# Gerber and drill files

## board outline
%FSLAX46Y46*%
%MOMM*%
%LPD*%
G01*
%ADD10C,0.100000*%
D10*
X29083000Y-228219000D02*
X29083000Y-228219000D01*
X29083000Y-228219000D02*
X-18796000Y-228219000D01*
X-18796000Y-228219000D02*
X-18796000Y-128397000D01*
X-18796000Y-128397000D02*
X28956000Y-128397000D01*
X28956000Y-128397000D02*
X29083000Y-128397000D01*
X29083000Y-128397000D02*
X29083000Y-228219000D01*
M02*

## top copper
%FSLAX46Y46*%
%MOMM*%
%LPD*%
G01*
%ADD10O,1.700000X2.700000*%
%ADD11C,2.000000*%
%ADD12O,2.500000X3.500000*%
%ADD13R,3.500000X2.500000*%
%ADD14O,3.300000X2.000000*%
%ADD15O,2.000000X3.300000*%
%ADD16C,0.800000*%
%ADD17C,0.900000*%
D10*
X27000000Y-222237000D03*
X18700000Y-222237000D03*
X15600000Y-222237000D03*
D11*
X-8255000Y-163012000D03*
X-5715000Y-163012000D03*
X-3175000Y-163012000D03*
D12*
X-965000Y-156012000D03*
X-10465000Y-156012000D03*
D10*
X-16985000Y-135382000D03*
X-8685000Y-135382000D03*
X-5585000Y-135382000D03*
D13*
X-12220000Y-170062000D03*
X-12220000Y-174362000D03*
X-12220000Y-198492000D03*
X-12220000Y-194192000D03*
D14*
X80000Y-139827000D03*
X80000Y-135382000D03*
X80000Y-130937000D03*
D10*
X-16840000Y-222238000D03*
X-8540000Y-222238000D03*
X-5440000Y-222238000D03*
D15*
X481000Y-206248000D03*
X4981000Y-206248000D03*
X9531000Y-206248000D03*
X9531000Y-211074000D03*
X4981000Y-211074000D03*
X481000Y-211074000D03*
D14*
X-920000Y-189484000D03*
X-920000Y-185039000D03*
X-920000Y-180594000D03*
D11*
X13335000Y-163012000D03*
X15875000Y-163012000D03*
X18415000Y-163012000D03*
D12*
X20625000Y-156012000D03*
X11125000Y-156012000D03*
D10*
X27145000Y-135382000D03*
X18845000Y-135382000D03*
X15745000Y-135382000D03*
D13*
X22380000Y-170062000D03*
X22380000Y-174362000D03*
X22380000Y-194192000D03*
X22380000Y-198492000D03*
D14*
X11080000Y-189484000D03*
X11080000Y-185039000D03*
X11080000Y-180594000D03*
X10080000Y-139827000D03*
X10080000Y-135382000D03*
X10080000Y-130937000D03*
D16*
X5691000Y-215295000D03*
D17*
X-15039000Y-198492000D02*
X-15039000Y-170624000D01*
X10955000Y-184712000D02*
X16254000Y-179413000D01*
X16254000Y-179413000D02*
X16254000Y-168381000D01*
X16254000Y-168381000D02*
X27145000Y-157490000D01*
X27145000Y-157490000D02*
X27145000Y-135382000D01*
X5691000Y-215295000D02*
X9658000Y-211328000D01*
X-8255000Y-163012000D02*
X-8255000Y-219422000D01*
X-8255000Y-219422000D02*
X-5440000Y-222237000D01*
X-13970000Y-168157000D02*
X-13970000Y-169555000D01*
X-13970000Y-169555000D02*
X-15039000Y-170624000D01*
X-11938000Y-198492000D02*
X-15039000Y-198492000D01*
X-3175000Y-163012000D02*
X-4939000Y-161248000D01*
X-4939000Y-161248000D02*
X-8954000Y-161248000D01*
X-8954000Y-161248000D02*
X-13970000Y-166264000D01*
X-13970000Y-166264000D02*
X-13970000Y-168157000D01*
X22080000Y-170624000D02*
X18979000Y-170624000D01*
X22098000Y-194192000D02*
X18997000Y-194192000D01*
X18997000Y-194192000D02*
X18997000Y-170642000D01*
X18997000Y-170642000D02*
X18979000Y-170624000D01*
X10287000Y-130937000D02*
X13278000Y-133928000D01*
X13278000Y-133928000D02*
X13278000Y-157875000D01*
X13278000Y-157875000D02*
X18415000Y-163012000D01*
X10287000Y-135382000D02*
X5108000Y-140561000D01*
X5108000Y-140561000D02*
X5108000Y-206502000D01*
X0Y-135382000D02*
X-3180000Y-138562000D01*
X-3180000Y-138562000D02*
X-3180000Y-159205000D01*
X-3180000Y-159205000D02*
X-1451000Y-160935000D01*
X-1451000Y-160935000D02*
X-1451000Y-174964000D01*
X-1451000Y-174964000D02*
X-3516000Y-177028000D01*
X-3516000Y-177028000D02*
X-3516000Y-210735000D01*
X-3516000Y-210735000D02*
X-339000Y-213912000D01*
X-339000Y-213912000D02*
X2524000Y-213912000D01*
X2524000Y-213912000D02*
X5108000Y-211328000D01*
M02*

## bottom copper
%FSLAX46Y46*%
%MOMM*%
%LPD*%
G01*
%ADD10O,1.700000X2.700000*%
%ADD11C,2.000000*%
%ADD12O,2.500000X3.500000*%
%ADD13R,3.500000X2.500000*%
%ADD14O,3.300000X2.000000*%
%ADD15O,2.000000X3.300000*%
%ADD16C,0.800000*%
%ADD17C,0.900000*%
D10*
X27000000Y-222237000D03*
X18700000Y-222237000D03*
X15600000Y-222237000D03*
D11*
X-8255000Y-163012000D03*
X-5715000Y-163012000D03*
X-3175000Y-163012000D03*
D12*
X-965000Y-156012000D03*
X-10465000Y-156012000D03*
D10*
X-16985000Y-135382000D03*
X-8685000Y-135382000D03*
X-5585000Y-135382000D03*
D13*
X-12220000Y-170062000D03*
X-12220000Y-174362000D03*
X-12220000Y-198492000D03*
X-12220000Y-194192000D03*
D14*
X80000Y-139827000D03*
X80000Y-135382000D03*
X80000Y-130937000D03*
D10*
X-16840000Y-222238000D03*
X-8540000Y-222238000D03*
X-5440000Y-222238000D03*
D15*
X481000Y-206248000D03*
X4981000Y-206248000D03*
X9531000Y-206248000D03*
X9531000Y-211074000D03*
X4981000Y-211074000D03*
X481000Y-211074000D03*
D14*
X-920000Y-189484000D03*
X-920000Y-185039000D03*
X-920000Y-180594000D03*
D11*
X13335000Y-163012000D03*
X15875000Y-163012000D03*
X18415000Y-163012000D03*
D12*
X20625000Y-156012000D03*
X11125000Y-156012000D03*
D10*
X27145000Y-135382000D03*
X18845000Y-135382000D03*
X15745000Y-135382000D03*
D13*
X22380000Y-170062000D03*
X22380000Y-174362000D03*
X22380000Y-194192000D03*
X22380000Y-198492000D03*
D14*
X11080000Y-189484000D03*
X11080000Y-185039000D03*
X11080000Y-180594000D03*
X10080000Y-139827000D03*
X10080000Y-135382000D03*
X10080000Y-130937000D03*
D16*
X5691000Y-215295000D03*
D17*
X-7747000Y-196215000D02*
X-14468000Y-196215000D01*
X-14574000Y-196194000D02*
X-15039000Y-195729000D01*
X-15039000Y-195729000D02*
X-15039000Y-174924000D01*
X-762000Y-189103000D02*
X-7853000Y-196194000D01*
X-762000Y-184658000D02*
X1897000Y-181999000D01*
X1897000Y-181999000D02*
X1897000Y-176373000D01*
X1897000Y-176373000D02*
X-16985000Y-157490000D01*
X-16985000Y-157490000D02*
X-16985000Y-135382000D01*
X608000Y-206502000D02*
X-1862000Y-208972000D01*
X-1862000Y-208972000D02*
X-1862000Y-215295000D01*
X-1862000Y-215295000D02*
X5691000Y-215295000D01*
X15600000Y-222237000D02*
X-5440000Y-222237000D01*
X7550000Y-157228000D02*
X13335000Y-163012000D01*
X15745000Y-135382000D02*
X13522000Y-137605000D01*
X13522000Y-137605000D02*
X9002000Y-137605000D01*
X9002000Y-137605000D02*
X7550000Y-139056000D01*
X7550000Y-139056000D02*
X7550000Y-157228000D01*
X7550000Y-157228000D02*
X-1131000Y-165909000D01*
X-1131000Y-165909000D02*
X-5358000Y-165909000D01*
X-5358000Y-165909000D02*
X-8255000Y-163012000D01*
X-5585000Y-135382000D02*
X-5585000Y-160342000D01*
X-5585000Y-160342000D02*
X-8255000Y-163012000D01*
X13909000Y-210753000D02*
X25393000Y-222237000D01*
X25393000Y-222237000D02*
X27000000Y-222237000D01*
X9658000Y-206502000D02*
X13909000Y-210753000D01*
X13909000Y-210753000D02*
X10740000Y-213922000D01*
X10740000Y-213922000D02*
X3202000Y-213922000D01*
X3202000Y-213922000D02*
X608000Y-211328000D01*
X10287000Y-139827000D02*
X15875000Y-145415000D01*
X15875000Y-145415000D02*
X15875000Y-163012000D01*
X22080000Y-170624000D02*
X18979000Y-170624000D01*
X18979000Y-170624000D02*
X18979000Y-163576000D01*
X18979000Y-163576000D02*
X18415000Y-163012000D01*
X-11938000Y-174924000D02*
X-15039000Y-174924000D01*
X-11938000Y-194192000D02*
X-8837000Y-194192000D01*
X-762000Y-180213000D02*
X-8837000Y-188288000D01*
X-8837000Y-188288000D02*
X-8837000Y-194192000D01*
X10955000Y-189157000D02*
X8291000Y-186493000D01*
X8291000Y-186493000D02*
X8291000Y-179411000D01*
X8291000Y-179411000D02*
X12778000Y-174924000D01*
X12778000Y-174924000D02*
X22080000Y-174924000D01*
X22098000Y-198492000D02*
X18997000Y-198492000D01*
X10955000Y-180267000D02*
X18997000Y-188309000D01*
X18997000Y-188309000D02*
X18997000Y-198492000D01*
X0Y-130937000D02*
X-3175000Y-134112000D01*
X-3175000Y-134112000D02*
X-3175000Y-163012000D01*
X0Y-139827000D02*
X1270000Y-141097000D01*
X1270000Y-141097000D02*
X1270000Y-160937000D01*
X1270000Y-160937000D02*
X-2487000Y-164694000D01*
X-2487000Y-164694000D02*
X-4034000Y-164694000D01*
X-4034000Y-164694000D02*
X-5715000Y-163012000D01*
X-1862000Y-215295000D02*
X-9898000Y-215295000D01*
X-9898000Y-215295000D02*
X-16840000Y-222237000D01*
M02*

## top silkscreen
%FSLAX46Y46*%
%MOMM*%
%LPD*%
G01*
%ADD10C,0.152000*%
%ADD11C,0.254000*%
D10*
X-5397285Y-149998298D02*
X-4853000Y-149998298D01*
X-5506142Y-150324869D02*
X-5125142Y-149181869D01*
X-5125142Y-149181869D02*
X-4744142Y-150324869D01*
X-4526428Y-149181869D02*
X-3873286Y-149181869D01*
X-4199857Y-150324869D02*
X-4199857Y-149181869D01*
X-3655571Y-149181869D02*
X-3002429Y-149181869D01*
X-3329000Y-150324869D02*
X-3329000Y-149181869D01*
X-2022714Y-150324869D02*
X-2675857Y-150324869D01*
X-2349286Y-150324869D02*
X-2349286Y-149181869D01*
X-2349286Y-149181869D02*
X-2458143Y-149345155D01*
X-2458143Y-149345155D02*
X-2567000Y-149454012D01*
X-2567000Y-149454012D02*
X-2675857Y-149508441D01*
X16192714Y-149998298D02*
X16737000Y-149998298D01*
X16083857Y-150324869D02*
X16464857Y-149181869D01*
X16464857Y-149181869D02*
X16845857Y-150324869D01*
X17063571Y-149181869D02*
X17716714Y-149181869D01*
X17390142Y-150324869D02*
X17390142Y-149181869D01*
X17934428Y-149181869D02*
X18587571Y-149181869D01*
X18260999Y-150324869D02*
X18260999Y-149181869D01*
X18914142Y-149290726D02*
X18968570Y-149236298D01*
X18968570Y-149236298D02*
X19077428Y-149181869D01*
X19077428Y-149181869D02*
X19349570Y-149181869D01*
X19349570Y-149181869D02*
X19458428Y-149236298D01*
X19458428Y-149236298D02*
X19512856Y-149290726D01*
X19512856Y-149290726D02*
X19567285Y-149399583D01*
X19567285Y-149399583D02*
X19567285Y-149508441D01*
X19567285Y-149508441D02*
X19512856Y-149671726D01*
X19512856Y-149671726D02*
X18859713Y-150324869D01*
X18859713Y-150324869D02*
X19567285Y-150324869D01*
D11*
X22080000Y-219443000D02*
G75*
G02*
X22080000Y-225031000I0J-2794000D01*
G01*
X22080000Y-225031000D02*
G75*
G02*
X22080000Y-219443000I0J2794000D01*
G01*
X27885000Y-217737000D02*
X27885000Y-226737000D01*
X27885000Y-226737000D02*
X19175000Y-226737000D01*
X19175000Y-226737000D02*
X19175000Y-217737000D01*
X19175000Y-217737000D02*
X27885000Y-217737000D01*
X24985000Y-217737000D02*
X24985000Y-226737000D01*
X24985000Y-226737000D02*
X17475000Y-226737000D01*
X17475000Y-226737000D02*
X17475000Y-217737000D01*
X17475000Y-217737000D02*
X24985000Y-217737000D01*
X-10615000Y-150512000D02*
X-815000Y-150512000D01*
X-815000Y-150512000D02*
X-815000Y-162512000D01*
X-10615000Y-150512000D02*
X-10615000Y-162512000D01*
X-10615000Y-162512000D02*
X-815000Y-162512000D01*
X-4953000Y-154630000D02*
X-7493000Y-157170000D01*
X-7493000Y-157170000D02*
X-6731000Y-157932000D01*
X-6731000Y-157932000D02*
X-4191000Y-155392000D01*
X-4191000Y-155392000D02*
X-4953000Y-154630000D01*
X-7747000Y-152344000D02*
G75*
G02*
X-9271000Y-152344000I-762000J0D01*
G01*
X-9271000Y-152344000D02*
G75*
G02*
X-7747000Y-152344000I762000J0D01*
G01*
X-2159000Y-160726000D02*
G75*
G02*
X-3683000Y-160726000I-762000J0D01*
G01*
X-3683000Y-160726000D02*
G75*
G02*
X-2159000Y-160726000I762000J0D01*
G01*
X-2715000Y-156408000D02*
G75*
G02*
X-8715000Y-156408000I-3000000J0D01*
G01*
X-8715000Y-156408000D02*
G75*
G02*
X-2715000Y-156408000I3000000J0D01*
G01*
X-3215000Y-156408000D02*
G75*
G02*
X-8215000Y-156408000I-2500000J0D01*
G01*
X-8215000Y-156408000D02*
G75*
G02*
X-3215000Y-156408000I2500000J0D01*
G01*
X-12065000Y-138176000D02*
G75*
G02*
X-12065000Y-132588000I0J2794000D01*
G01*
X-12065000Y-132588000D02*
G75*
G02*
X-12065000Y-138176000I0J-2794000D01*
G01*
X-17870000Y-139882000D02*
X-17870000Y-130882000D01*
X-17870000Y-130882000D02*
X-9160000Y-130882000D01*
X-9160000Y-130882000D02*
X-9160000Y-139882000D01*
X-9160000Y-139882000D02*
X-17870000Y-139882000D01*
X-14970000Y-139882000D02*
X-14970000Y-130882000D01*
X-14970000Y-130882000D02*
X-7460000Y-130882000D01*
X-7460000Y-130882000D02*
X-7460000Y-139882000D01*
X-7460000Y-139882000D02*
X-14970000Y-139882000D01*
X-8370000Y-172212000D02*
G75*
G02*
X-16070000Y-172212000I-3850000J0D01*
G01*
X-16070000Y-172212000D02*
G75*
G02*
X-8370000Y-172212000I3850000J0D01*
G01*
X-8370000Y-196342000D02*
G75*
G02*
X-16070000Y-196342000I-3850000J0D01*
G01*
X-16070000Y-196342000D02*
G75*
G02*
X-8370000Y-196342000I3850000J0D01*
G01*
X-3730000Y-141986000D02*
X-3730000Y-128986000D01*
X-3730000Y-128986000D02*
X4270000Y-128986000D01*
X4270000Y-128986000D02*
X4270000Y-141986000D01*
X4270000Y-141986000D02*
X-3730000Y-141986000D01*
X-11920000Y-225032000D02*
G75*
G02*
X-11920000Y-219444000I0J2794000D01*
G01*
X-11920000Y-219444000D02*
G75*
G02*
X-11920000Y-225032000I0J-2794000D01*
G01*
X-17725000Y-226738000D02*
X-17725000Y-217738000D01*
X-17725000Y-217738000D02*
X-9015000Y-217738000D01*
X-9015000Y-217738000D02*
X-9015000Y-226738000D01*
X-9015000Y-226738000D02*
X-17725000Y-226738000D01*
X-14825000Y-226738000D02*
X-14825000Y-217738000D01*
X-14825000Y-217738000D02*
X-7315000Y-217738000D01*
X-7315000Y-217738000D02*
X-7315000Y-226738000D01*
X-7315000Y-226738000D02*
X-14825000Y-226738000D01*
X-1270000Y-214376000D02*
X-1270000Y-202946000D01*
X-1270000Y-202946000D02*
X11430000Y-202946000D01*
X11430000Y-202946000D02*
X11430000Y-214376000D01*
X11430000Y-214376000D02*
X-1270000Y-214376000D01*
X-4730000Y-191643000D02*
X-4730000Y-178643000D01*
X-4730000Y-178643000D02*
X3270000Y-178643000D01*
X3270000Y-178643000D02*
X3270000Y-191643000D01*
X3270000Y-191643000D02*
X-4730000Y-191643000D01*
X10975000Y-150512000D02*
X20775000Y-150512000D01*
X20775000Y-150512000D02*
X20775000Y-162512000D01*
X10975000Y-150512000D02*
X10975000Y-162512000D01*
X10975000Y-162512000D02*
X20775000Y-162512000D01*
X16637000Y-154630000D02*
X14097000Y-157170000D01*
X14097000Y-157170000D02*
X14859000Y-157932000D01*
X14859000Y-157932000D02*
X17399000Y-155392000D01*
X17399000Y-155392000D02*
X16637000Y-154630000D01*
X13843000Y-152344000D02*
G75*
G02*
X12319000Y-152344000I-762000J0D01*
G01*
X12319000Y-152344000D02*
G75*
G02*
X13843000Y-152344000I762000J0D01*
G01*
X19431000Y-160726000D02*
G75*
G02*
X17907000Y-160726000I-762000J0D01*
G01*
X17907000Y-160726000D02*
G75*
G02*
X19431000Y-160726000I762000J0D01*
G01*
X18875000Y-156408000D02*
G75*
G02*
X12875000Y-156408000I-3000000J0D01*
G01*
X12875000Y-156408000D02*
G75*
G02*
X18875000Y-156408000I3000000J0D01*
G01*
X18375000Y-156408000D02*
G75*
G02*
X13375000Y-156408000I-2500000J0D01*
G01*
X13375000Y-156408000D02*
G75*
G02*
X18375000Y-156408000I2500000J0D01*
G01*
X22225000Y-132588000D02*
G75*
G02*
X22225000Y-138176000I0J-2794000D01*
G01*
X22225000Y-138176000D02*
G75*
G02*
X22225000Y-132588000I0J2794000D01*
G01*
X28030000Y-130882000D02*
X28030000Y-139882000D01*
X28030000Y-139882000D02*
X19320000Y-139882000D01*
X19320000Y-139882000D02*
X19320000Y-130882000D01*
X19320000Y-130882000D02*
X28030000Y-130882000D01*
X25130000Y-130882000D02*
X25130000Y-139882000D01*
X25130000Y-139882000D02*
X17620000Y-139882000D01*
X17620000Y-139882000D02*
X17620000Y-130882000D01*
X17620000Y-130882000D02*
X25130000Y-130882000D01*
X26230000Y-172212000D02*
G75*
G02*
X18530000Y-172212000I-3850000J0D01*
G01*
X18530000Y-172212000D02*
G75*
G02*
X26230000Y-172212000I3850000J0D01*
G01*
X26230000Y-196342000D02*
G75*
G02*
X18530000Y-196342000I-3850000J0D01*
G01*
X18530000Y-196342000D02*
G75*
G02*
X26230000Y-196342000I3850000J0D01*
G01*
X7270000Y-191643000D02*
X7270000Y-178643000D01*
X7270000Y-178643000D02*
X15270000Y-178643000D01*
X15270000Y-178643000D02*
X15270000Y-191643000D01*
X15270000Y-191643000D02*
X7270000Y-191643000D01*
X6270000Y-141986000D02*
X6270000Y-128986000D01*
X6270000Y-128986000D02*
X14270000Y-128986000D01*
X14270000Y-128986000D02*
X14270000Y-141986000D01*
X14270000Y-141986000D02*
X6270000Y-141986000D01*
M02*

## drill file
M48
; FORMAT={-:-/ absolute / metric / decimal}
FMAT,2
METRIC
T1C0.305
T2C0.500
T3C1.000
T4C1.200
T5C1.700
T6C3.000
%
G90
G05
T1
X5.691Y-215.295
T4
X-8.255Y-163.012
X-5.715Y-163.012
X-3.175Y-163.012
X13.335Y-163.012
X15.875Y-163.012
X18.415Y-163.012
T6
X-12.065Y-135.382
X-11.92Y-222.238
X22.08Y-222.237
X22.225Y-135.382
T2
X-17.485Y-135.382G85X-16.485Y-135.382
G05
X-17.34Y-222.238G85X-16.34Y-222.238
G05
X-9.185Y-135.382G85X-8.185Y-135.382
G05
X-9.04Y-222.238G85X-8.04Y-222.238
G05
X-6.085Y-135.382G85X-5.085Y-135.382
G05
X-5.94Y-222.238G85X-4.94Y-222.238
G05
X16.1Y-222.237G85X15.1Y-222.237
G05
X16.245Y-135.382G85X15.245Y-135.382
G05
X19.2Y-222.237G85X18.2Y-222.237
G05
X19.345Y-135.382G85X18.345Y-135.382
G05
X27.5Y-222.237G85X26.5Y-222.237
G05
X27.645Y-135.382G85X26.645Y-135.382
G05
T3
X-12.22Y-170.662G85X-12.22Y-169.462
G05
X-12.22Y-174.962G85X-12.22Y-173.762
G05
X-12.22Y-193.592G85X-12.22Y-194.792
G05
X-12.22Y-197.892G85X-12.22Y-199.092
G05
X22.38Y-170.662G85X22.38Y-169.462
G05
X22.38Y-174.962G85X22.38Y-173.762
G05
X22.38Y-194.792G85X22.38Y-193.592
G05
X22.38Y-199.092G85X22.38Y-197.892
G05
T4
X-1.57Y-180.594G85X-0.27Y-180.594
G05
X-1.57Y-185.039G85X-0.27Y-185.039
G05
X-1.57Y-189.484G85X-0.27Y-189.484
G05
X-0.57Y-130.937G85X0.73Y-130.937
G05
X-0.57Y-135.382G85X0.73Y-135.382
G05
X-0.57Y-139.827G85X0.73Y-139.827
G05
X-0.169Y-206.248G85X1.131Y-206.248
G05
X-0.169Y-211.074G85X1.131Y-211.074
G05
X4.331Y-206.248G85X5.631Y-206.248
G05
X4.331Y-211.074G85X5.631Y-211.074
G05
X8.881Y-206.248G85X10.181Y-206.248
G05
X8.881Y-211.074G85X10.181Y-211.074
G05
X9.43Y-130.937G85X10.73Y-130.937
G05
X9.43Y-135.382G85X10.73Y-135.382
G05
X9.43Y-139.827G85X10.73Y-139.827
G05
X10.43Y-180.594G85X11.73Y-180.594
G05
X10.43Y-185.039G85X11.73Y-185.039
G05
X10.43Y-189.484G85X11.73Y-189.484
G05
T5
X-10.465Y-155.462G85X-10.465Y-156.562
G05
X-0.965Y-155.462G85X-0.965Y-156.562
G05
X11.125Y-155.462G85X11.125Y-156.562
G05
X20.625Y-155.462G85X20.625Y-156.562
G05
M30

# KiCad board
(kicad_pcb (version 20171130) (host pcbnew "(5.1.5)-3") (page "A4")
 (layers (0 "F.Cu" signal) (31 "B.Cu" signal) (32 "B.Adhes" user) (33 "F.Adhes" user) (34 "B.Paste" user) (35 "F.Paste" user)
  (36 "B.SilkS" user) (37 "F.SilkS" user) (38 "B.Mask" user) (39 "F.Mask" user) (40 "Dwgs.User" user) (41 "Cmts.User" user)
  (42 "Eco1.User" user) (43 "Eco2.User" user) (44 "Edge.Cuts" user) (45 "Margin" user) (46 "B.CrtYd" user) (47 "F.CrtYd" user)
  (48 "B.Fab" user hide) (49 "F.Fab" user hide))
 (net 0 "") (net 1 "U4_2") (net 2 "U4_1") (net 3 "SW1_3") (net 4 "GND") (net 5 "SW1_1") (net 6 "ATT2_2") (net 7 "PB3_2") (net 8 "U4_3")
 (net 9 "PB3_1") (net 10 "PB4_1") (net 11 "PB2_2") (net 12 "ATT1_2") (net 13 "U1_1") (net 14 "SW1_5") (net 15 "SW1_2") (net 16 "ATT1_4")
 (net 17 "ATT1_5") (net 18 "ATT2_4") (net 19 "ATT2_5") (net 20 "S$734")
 (segment (start -7.747 196.215) (end -14.468 196.215) (width 0.9) (layer "B.Cu") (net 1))
 (segment (start -14.574 196.194) (end -15.039 195.729) (width 0.9) (layer "B.Cu") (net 1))
 (segment (start -15.039 195.729) (end -15.039 174.924) (width 0.9) (layer "B.Cu") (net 1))
 (segment (start -0.762 189.103) (end -7.853 196.194) (width 0.9) (layer "B.Cu") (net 1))
 (segment (start -0.762 184.658) (end 1.897 181.999) (width 0.9) (layer "B.Cu") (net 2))
 (segment (start 1.897 181.999) (end 1.897 176.373) (width 0.9) (layer "B.Cu") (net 2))
 (segment (start 1.897 176.373) (end -16.985 157.49) (width 0.9) (layer "B.Cu") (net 2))
 (segment (start -16.985 157.49) (end -16.985 135.382) (width 0.9) (layer "B.Cu") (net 2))
 (segment (start 0.608 206.502) (end -1.862 208.972) (width 0.9) (layer "B.Cu") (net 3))
 (segment (start -1.862 208.972) (end -1.862 215.295) (width 0.9) (layer "B.Cu") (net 3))
 (segment (start -1.862 215.295) (end 5.691 215.295) (width 0.9) (layer "B.Cu") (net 3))
 (segment (start 15.6 222.237) (end -5.44 222.237) (width 0.9) (layer "B.Cu") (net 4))
 (segment (start 7.55 157.228) (end 13.335 163.012) (width 0.9) (layer "B.Cu") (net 4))
 (segment (start 15.745 135.382) (end 13.522 137.605) (width 0.9) (layer "B.Cu") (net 4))
 (segment (start 13.522 137.605) (end 9.002 137.605) (width 0.9) (layer "B.Cu") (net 4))
 (segment (start 9.002 137.605) (end 7.55 139.056) (width 0.9) (layer "B.Cu") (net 4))
 (segment (start 7.55 139.056) (end 7.55 157.228) (width 0.9) (layer "B.Cu") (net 4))
 (segment (start 7.55 157.228) (end -1.131 165.909) (width 0.9) (layer "B.Cu") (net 4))
 (segment (start -1.131 165.909) (end -5.358 165.909) (width 0.9) (layer "B.Cu") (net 4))
 (segment (start -5.358 165.909) (end -8.255 163.012) (width 0.9) (layer "B.Cu") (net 4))
 (segment (start -5.585 135.382) (end -5.585 160.342) (width 0.9) (layer "B.Cu") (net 4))
 (segment (start -5.585 160.342) (end -8.255 163.012) (width 0.9) (layer "B.Cu") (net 4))
 (segment (start 13.909 210.753) (end 25.393 222.237) (width 0.9) (layer "B.Cu") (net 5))
 (segment (start 25.393 222.237) (end 27 222.237) (width 0.9) (layer "B.Cu") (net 5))
 (segment (start 9.658 206.502) (end 13.909 210.753) (width 0.9) (layer "B.Cu") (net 5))
 (segment (start 13.909 210.753) (end 10.74 213.922) (width 0.9) (layer "B.Cu") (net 5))
 (segment (start 10.74 213.922) (end 3.202 213.922) (width 0.9) (layer "B.Cu") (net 5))
 (segment (start 3.202 213.922) (end 0.608 211.328) (width 0.9) (layer "B.Cu") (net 5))
 (segment (start 10.287 139.827) (end 15.875 145.415) (width 0.9) (layer "B.Cu") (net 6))
 (segment (start 15.875 145.415) (end 15.875 163.012) (width 0.9) (layer "B.Cu") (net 6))
 (segment (start 22.08 170.624) (end 18.979 170.624) (width 0.9) (layer "B.Cu") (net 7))
 (segment (start 18.979 170.624) (end 18.979 163.576) (width 0.9) (layer "B.Cu") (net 7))
 (segment (start 18.979 163.576) (end 18.415 163.012) (width 0.9) (layer "B.Cu") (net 7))
 (segment (start -11.938 174.924) (end -15.039 174.924) (width 0.9) (layer "B.Cu") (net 1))
 (segment (start -11.938 194.192) (end -8.837 194.192) (width 0.9) (layer "B.Cu") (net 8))
 (segment (start -0.762 180.213) (end -8.837 188.288) (width 0.9) (layer "B.Cu") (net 8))
 (segment (start -8.837 188.288) (end -8.837 194.192) (width 0.9) (layer "B.Cu") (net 8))
 (segment (start 10.955 189.157) (end 8.291 186.493) (width 0.9) (layer "B.Cu") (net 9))
 (segment (start 8.291 186.493) (end 8.291 179.411) (width 0.9) (layer "B.Cu") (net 9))
 (segment (start 8.291 179.411) (end 12.778 174.924) (width 0.9) (layer "B.Cu") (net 9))
 (segment (start 12.778 174.924) (end 22.08 174.924) (width 0.9) (layer "B.Cu") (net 9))
 (segment (start 22.098 198.492) (end 18.997 198.492) (width 0.9) (layer "B.Cu") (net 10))
 (segment (start 10.955 180.267) (end 18.997 188.309) (width 0.9) (layer "B.Cu") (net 10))
 (segment (start 18.997 188.309) (end 18.997 198.492) (width 0.9) (layer "B.Cu") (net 10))
 (segment (start 0 130.937) (end -3.175 134.112) (width 0.9) (layer "B.Cu") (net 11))
 (segment (start -3.175 134.112) (end -3.175 163.012) (width 0.9) (layer "B.Cu") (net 11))
 (segment (start 0 139.827) (end 1.27 141.097) (width 0.9) (layer "B.Cu") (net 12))
 (segment (start 1.27 141.097) (end 1.27 160.937) (width 0.9) (layer "B.Cu") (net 12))
 (segment (start 1.27 160.937) (end -2.487 164.694) (width 0.9) (layer "B.Cu") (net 12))
 (segment (start -2.487 164.694) (end -4.034 164.694) (width 0.9) (layer "B.Cu") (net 12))
 (segment (start -4.034 164.694) (end -5.715 163.012) (width 0.9) (layer "B.Cu") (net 12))
 (segment (start -1.862 215.295) (end -9.898 215.295) (width 0.9) (layer "B.Cu") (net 3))
 (segment (start -9.898 215.295) (end -16.84 222.237) (width 0.9) (layer "B.Cu") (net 3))
 (gr_line (start 29.083 228.219) (end 29.083 228.219) (width 0.1) (layer "Edge.Cuts"))
 (gr_line (start 29.083 228.219) (end -18.796 228.219) (width 0.1) (layer "Edge.Cuts"))
 (gr_line (start -18.796 228.219) (end -18.796 128.397) (width 0.1) (layer "Edge.Cuts"))
 (gr_line (start -18.796 128.397) (end 28.956 128.397) (width 0.1) (layer "Edge.Cuts"))
 (gr_line (start 28.956 128.397) (end 29.083 128.397) (width 0.1) (layer "Edge.Cuts"))
 (gr_line (start 29.083 128.397) (end 29.083 228.219) (width 0.1) (layer "Edge.Cuts"))
 (segment (start -15.039 198.492) (end -15.039 170.624) (width 0.9) (layer "F.Cu") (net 11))
 (segment (start 10.955 184.712) (end 16.254 179.413) (width 0.9) (layer "F.Cu") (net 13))
 (segment (start 16.254 179.413) (end 16.254 168.381) (width 0.9) (layer "F.Cu") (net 13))
 (segment (start 16.254 168.381) (end 27.145 157.49) (width 0.9) (layer "F.Cu") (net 13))
 (segment (start 27.145 157.49) (end 27.145 135.382) (width 0.9) (layer "F.Cu") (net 13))
 (segment (start 5.691 215.295) (end 9.658 211.328) (width 0.9) (layer "F.Cu") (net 3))
 (segment (start -8.255 163.012) (end -8.255 219.422) (width 0.9) (layer "F.Cu") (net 4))
 (segment (start -8.255 219.422) (end -5.44 222.237) (width 0.9) (layer "F.Cu") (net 4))
 (segment (start -13.97 168.157) (end -13.97 169.555) (width 0.9) (layer "F.Cu") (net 11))
 (segment (start -13.97 169.555) (end -15.039 170.624) (width 0.9) (layer "F.Cu") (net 11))
 (segment (start -11.938 198.492) (end -15.039 198.492) (width 0.9) (layer "F.Cu") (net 11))
 (segment (start -3.175 163.012) (end -4.939 161.248) (width 0.9) (layer "F.Cu") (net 11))
 (segment (start -4.939 161.248) (end -8.954 161.248) (width 0.9) (layer "F.Cu") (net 11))
 (segment (start -8.954 161.248) (end -13.97 166.264) (width 0.9) (layer "F.Cu") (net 11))
 (segment (start -13.97 166.264) (end -13.97 168.157) (width 0.9) (layer "F.Cu") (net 11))
 (segment (start 22.08 170.624) (end 18.979 170.624) (width 0.9) (layer "F.Cu") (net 7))
 (segment (start 22.098 194.192) (end 18.997 194.192) (width 0.9) (layer "F.Cu") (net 7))
 (segment (start 18.997 194.192) (end 18.997 170.642) (width 0.9) (layer "F.Cu") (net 7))
 (segment (start 18.997 170.642) (end 18.979 170.624) (width 0.9) (layer "F.Cu") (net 7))
 (segment (start 10.287 130.937) (end 13.278 133.928) (width 0.9) (layer "F.Cu") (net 7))
 (segment (start 13.278 133.928) (end 13.278 157.875) (width 0.9) (layer "F.Cu") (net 7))
 (segment (start 13.278 157.875) (end 18.415 163.012) (width 0.9) (layer "F.Cu") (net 7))
 (segment (start 10.287 135.382) (end 5.108 140.561) (width 0.9) (layer "F.Cu") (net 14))
 (segment (start 5.108 140.561) (end 5.108 206.502) (width 0.9) (layer "F.Cu") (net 14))
 (segment (start 0 135.382) (end -3.18 138.562) (width 0.9) (layer "F.Cu") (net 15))
 (segment (start -3.18 138.562) (end -3.18 159.205) (width 0.9) (layer "F.Cu") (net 15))
 (segment (start -3.18 159.205) (end -1.451 160.935) (width 0.9) (layer "F.Cu") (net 15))
 (segment (start -1.451 160.935) (end -1.451 174.964) (width 0.9) (layer "F.Cu") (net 15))
 (segment (start -1.451 174.964) (end -3.516 177.028) (width 0.9) (layer "F.Cu") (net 15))
 (segment (start -3.516 177.028) (end -3.516 210.735) (width 0.9) (layer "F.Cu") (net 15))
 (segment (start -3.516 210.735) (end -0.339 213.912) (width 0.9) (layer "F.Cu") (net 15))
 (segment (start -0.339 213.912) (end 2.524 213.912) (width 0.9) (layer "F.Cu") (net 15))
 (segment (start 2.524 213.912) (end 5.108 211.328) (width 0.9) (layer "F.Cu") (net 15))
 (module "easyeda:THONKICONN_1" (layer "F.Cu") (at 22.08 222.237 -90)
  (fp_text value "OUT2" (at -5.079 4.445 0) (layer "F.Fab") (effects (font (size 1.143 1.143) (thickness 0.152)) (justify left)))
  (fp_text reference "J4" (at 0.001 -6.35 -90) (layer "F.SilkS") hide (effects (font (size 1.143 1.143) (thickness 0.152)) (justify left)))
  (fp_arc (start 0 0) (end -2.794 0) (angle 180) (width 0.254) (layer "F.SilkS"))
  (fp_arc (start 0 0) (end 2.794 0) (angle 180) (width 0.254) (layer "F.SilkS"))
  (fp_line (start -4.5 -5.805) (end 4.5 -5.805) (width 0.254) (layer "F.SilkS"))
  (fp_line (start 4.5 -5.805) (end 4.5 2.905) (width 0.254) (layer "F.SilkS"))
  (fp_line (start 4.5 2.905) (end -4.5 2.905) (width 0.254) (layer "F.SilkS"))
  (fp_line (start -4.5 2.905) (end -4.5 -5.805) (width 0.254) (layer "F.SilkS"))
  (fp_line (start -4.5 -2.905) (end 4.5 -2.905) (width 0.254) (layer "F.SilkS"))
  (fp_line (start 4.5 -2.905) (end 4.5 4.605) (width 0.254) (layer "F.SilkS"))
  (fp_line (start 4.5 4.605) (end -4.5 4.605) (width 0.254) (layer "F.SilkS"))
  (fp_line (start -4.5 4.605) (end -4.5 -2.905) (width 0.254) (layer "F.SilkS"))
  (pad "" np_thru_hole circle (at 0 0) (size 3 3) (drill 3) (layers "*.Cu" "*.Mask"))
  (pad 3 thru_hole oval (at 0 -4.92 -90) (size 2.7 1.7) (layers "*.Cu" "*.Paste" "*.Mask") (drill oval 0.5 1.5) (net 5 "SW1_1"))
  (pad 2 thru_hole oval (at 0 3.38 -90) (size 2.7 1.7) (layers "*.Cu" "*.Paste" "*.Mask") (drill oval 0.5 1.5))
  (pad 1 thru_hole oval (at 0 6.48 -90) (size 2.7 1.7) (layers "*.Cu" "*.Paste" "*.Mask") (drill oval 0.5 1.5) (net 4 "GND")))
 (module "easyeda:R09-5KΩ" (layer "F.Cu") (at -5.715 159.512)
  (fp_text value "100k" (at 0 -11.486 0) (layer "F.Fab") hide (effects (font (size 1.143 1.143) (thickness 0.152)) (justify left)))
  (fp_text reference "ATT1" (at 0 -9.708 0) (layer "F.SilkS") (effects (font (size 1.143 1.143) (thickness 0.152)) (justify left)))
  (fp_line (start -4.9 -9) (end 4.9 -9) (width 0.254) (layer "F.SilkS"))
  (fp_line (start 4.9 -9) (end 4.9 3) (width 0.254) (layer "F.SilkS"))
  (fp_line (start -4.9 -9) (end -4.9 3) (width 0.254) (layer "F.SilkS"))
  (fp_line (start -4.9 3) (end 4.9 3) (width 0.254) (layer "F.SilkS"))
  (fp_line (start 0.762 -4.882) (end -1.778 -2.342) (width 0.254) (layer "F.SilkS"))
  (fp_line (start -1.778 -2.342) (end -1.016 -1.58) (width 0.254) (layer "F.SilkS"))
  (fp_line (start -1.016 -1.58) (end 1.524 -4.12) (width 0.254) (layer "F.SilkS"))
  (fp_line (start 1.524 -4.12) (end 0.762 -4.882) (width 0.254) (layer "F.SilkS"))
  (fp_circle (center -2.794 -7.168) (end -2.032 -7.168) (layer "F.SilkS") (width 0.254))
  (fp_circle (center 2.794 1.214) (end 3.556 1.214) (layer "F.SilkS") (width 0.254))
  (fp_circle (center 0 -3.104) (end 3 -3.104) (layer "F.SilkS") (width 0.254))
  (fp_circle (center 0 -3.104) (end 2.5 -3.104) (layer "F.SilkS") (width 0.254))
  (pad 1 thru_hole circle (at -2.54 3.5 0) (size 2 2) (layers "*.Cu" "*.Paste" "*.Mask") (drill 1.2) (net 4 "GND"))
  (pad 2 thru_hole circle (at 0 3.5 0) (size 2 2) (layers "*.Cu" "*.Paste" "*.Mask") (drill 1.2) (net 12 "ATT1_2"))
  (pad 3 thru_hole circle (at 2.54 3.5 0) (size 2 2) (layers "*.Cu" "*.Paste" "*.Mask") (drill 1.2) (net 11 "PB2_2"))
  (pad 4 thru_hole oval (at 4.75 -3.5 0) (size 2.5 3.5) (layers "*.Cu" "*.Paste" "*.Mask") (drill oval 1.7 2.8) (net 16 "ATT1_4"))
  (pad 5 thru_hole oval (at -4.75 -3.5 0) (size 2.5 3.5) (layers "*.Cu" "*.Paste" "*.Mask") (drill oval 1.7 2.8) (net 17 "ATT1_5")))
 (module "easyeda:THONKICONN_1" (layer "F.Cu") (at -12.065 135.382 90)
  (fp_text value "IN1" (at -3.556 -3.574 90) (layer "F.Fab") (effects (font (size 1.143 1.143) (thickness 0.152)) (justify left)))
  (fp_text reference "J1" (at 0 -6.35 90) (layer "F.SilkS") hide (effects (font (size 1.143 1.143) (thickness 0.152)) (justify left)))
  (fp_arc (start 0 0) (end -2.794 0) (angle 180) (width 0.254) (layer "F.SilkS"))
  (fp_arc (start 0 0) (end 2.794 0) (angle 180) (width 0.254) (layer "F.SilkS"))
  (pad "" np_thru_hole circle (at 0 0) (size 3 3) (drill 3) (layers "*.Cu" "*.Mask"))
  (fp_line (start -4.5 -5.805) (end 4.5 -5.805) (width 0.254) (layer "F.SilkS"))
  (fp_line (start 4.5 -5.805) (end 4.5 2.905) (width 0.254) (layer "F.SilkS"))
  (fp_line (start 4.5 2.905) (end -4.5 2.905) (width 0.254) (layer "F.SilkS"))
  (fp_line (start -4.5 2.905) (end -4.5 -5.805) (width 0.254) (layer "F.SilkS"))
  (fp_line (start -4.5 -2.905) (end 4.5 -2.905) (width 0.254) (layer "F.SilkS"))
  (fp_line (start 4.5 -2.905) (end 4.5 4.605) (width 0.254) (layer "F.SilkS"))
  (fp_line (start 4.5 4.605) (end -4.5 4.605) (width 0.254) (layer "F.SilkS"))
  (fp_line (start -4.5 4.605) (end -4.5 -2.905) (width 0.254) (layer "F.SilkS"))
  (pad 3 thru_hole oval (at 0 -4.92 90) (size 2.7 1.7) (layers "*.Cu" "*.Paste" "*.Mask") (drill oval 0.5 1.5) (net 2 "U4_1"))
  (pad 2 thru_hole oval (at 0 3.38 90) (size 2.7 1.7) (layers "*.Cu" "*.Paste" "*.Mask") (drill oval 0.5 1.5))
  (pad 1 thru_hole oval (at 0 6.48 90) (size 2.7 1.7) (layers "*.Cu" "*.Paste" "*.Mask") (drill oval 0.5 1.5) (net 4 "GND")))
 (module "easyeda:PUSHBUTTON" (layer "F.Cu") (at -12.22 172.212 90)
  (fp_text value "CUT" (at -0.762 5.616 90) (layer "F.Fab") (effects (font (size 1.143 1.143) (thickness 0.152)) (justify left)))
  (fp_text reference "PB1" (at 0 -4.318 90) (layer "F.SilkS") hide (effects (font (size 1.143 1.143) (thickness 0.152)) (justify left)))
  (fp_circle (center 0 0) (end 3.85 0) (layer "F.SilkS") (width 0.254))
  (pad 2 thru_hole rect (at 2.15 0 180) (size 3.5 2.5) (layers "*.Cu" "*.Paste" "*.Mask") (drill oval 1 2.2) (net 11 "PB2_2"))
  (pad 1 thru_hole rect (at -2.15 0 180) (size 3.5 2.5) (layers "*.Cu" "*.Paste" "*.Mask") (drill oval 1 2.2) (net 1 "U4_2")))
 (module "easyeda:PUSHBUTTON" (layer "F.Cu") (at -12.22 196.342 -90)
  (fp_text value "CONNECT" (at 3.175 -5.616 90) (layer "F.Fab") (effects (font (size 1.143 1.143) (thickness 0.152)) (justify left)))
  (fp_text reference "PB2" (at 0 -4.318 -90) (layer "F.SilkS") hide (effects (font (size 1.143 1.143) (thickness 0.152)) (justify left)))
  (fp_circle (center 0 0) (end 3.85 0) (layer "F.SilkS") (width 0.254))
  (pad 2 thru_hole rect (at 2.15 0 0) (size 3.5 2.5) (layers "*.Cu" "*.Paste" "*.Mask") (drill oval 1 2.2) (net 11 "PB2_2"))
  (pad 1 thru_hole rect (at -2.15 0 0) (size 3.5 2.5) (layers "*.Cu" "*.Paste" "*.Mask") (drill oval 1 2.2) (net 8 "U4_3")))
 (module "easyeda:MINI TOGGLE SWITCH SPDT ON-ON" (layer "F.Cu") (at 0.08 135.382 90)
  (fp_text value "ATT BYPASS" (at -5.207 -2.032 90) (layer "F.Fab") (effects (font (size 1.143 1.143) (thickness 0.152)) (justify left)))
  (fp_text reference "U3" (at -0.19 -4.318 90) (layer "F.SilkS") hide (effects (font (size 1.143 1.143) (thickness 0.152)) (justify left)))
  (fp_line (start -6.604 -3.81) (end 6.396 -3.81) (width 0.254) (layer "F.SilkS") (status 40000))
  (fp_line (start 6.396 -3.81) (end 6.396 4.19) (width 0.254) (layer "F.SilkS") (status 40000))
  (fp_line (start 6.396 4.19) (end -6.604 4.19) (width 0.254) (layer "F.SilkS") (status 40000))
  (fp_line (start -6.604 4.19) (end -6.604 -3.81) (width 0.254) (layer "F.SilkS") (status 40000))
  (pad 2 thru_hole oval (at -4.445 0 90) (size 2 3.3) (layers "*.Cu" "*.Paste" "*.Mask") (drill oval 1.2 2.5) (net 12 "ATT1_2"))
  (pad 1 thru_hole oval (at 0 0 90) (size 2 3.3) (layers "*.Cu" "*.Paste" "*.Mask") (drill oval 1.2 2.5) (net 15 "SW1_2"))
  (pad 3 thru_hole oval (at 4.445 0 90) (size 2 3.3) (layers "*.Cu" "*.Paste" "*.Mask") (drill oval 1.2 2.5) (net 11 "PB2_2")))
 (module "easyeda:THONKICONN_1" (layer "F.Cu") (at -11.92 222.238 90)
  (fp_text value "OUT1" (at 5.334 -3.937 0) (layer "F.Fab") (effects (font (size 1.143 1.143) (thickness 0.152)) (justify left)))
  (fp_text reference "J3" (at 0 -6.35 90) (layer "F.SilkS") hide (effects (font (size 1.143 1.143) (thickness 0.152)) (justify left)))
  (fp_arc (start 0 0) (end -2.794 0) (angle 180) (width 0.254) (layer "F.SilkS"))
  (fp_arc (start 0 0) (end 2.794 0) (angle 180) (width 0.254) (layer "F.SilkS"))
  (fp_line (start -4.5 -5.805) (end 4.5 -5.805) (width 0.254) (layer "F.SilkS"))
  (fp_line (start 4.5 -5.805) (end 4.5 2.905) (width 0.254) (layer "F.SilkS"))
  (fp_line (start 4.5 2.905) (end -4.5 2.905) (width 0.254) (layer "F.SilkS"))
  (fp_line (start -4.5 2.905) (end -4.5 -5.805) (width 0.254) (layer "F.SilkS"))
  (fp_line (start -4.5 -2.905) (end 4.5 -2.905) (width 0.254) (layer "F.SilkS"))
  (fp_line (start 4.5 -2.905) (end 4.5 4.605) (width 0.254) (layer "F.SilkS"))
  (fp_line (start 4.5 4.605) (end -4.5 4.605) (width 0.254) (layer "F.SilkS"))
  (fp_line (start -4.5 4.605) (end -4.5 -2.905) (width 0.254) (layer "F.SilkS"))
  (pad "" np_thru_hole circle (at 0 0) (size 3 3) (drill 3) (layers "*.Cu" "*.Mask"))
  (pad 3 thru_hole oval (at 0 -4.92 90) (size 2.7 1.7) (layers "*.Cu" "*.Paste" "*.Mask") (drill oval 0.5 1.5) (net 3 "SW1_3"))
  (pad 2 thru_hole oval (at 0 3.38 90) (size 2.7 1.7) (layers "*.Cu" "*.Paste" "*.Mask") (drill oval 0.5 1.5))
  (pad 1 thru_hole oval (at 0 6.48 90) (size 2.7 1.7) (layers "*.Cu" "*.Paste" "*.Mask") (drill oval 0.5 1.5) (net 4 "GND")))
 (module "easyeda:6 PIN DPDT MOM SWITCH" (layer "F.Cu") (at 11.43 214.376 90)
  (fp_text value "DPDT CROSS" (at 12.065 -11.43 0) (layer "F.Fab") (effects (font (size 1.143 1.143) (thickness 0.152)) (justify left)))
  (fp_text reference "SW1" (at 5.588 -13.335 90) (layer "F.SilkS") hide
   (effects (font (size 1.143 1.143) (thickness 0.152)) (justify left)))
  (fp_line (start 0 -12.7) (end 11.43 -12.7) (width 0.254) (layer "F.SilkS"))
  (fp_line (start 11.43 -12.7) (end 11.43 0) (width 0.254) (layer "F.SilkS"))
  (fp_line (start 11.43 0) (end 0 0) (width 0.254) (layer "F.SilkS"))
  (fp_line (start 0 0) (end 0 -12.7) (width 0.254) (layer "F.SilkS"))
  (pad 4 thru_hole oval (at 8.128 -10.949 90) (size 3.3 2) (layers "*.Cu" "*.Paste" "*.Mask") (drill oval 1.2 2.5) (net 3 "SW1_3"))
  (pad 5 thru_hole oval (at 8.128 -6.449 90) (size 3.3 2) (layers "*.Cu" "*.Paste" "*.Mask") (drill oval 1.2 2.5) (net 14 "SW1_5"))
  (pad 6 thru_hole oval (at 8.128 -1.899 90) (size 3.3 2) (layers "*.Cu" "*.Paste" "*.Mask") (drill oval 1.2 2.5) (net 5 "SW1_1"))
  (pad 3 thru_hole oval (at 3.302 -1.899 90) (size 3.3 2) (layers "*.Cu" "*.Paste" "*.Mask") (drill oval 1.2 2.5) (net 3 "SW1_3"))
  (pad 2 thru_hole oval (at 3.302 -6.449 90) (size 3.3 2) (layers "*.Cu" "*.Paste" "*.Mask") (drill oval 1.2 2.5) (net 15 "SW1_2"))
  (pad 1 thru_hole oval (at 3.302 -10.949 90) (size 3.3 2) (layers "*.Cu" "*.Paste" "*.Mask") (drill oval 1.2 2.5) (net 5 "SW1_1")))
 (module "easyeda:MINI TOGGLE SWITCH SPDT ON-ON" (layer "F.Cu") (at -0.92 185.039 90)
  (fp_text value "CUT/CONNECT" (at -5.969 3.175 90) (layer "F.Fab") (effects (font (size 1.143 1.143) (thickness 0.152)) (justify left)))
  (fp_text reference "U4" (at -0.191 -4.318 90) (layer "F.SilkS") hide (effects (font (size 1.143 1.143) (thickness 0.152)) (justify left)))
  (fp_line (start -6.604 -3.81) (end 6.396 -3.81) (width 0.254) (layer "F.SilkS") (status 40000))
  (fp_line (start 6.396 -3.81) (end 6.396 4.19) (width 0.254) (layer "F.SilkS") (status 40000))
  (fp_line (start 6.396 4.19) (end -6.604 4.19) (width 0.254) (layer "F.SilkS") (status 40000))
  (fp_line (start -6.604 4.19) (end -6.604 -3.81) (width 0.254) (layer "F.SilkS") (status 40000))
  (pad 2 thru_hole oval (at -4.445 0 90) (size 2 3.3) (layers "*.Cu" "*.Paste" "*.Mask") (drill oval 1.2 2.5) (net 1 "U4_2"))
  (pad 1 thru_hole oval (at 0 0 90) (size 2 3.3) (layers "*.Cu" "*.Paste" "*.Mask") (drill oval 1.2 2.5) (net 2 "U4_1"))
  (pad 3 thru_hole oval (at 4.445 0 90) (size 2 3.3) (layers "*.Cu" "*.Paste" "*.Mask") (drill oval 1.2 2.5) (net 8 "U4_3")))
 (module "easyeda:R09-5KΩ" (layer "F.Cu") (at 15.875 159.512)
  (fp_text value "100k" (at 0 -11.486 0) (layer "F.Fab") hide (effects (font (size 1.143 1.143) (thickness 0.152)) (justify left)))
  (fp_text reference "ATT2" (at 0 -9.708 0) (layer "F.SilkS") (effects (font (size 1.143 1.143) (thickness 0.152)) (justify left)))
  (fp_line (start -4.9 -9) (end 4.9 -9) (width 0.254) (layer "F.SilkS"))
  (fp_line (start 4.9 -9) (end 4.9 3) (width 0.254) (layer "F.SilkS"))
  (fp_line (start -4.9 -9) (end -4.9 3) (width 0.254) (layer "F.SilkS"))
  (fp_line (start -4.9 3) (end 4.9 3) (width 0.254) (layer "F.SilkS"))
  (fp_line (start 0.762 -4.882) (end -1.778 -2.342) (width 0.254) (layer "F.SilkS"))
  (fp_line (start -1.778 -2.342) (end -1.016 -1.58) (width 0.254) (layer "F.SilkS"))
  (fp_line (start -1.016 -1.58) (end 1.524 -4.12) (width 0.254) (layer "F.SilkS"))
  (fp_line (start 1.524 -4.12) (end 0.762 -4.882) (width 0.254) (layer "F.SilkS"))
  (fp_circle (center -2.794 -7.168) (end -2.032 -7.168) (layer "F.SilkS") (width 0.254))
  (fp_circle (center 2.794 1.214) (end 3.556 1.214) (layer "F.SilkS") (width 0.254))
  (fp_circle (center 0 -3.104) (end 3 -3.104) (layer "F.SilkS") (width 0.254))
  (fp_circle (center 0 -3.104) (end 2.5 -3.104) (layer "F.SilkS") (width 0.254))
  (pad 1 thru_hole circle (at -2.54 3.5 0) (size 2 2) (layers "*.Cu" "*.Paste" "*.Mask") (drill 1.2) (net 4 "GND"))
  (pad 2 thru_hole circle (at 0 3.5 0) (size 2 2) (layers "*.Cu" "*.Paste" "*.Mask") (drill 1.2) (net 6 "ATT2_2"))
  (pad 3 thru_hole circle (at 2.54 3.5 0) (size 2 2) (layers "*.Cu" "*.Paste" "*.Mask") (drill 1.2) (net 7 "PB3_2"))
  (pad 4 thru_hole oval (at 4.75 -3.5 0) (size 2.5 3.5) (layers "*.Cu" "*.Paste" "*.Mask") (drill oval 1.7 2.8) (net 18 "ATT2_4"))
  (pad 5 thru_hole oval (at -4.75 -3.5 0) (size 2.5 3.5) (layers "*.Cu" "*.Paste" "*.Mask") (drill oval 1.7 2.8) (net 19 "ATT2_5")))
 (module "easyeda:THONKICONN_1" (layer "F.Cu") (at 22.225 135.382 -90)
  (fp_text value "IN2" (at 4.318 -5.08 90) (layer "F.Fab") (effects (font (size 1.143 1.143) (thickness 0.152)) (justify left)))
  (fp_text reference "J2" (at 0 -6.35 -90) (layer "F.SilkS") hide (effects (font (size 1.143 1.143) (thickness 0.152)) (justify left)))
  (fp_arc (start 0 0) (end -2.794 0) (angle 180) (width 0.254) (layer "F.SilkS"))
  (fp_arc (start 0 0) (end 2.794 0) (angle 180) (width 0.254) (layer "F.SilkS"))
  (pad "" np_thru_hole circle (at 0 0) (size 3 3) (drill 3) (layers "*.Cu" "*.Mask"))
  (fp_line (start -4.5 -5.805) (end 4.5 -5.805) (width 0.254) (layer "F.SilkS"))
  (fp_line (start 4.5 -5.805) (end 4.5 2.905) (width 0.254) (layer "F.SilkS"))
  (fp_line (start 4.5 2.905) (end -4.5 2.905) (width 0.254) (layer "F.SilkS"))
  (fp_line (start -4.5 2.905) (end -4.5 -5.805) (width 0.254) (layer "F.SilkS"))
  (fp_line (start -4.5 -2.905) (end 4.5 -2.905) (width 0.254) (layer "F.SilkS"))
  (fp_line (start 4.5 -2.905) (end 4.5 4.605) (width 0.254) (layer "F.SilkS"))
  (fp_line (start 4.5 4.605) (end -4.5 4.605) (width 0.254) (layer "F.SilkS"))
  (fp_line (start -4.5 4.605) (end -4.5 -2.905) (width 0.254) (layer "F.SilkS"))
  (pad 3 thru_hole oval (at 0 -4.92 -90) (size 2.7 1.7) (layers "*.Cu" "*.Paste" "*.Mask") (drill oval 0.5 1.5) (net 13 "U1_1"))
  (pad 2 thru_hole oval (at 0 3.38 -90) (size 2.7 1.7) (layers "*.Cu" "*.Paste" "*.Mask") (drill oval 0.5 1.5))
  (pad 1 thru_hole oval (at 0 6.48 -90) (size 2.7 1.7) (layers "*.Cu" "*.Paste" "*.Mask") (drill oval 0.5 1.5) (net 4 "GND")))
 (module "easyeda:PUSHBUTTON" (layer "F.Cu") (at 22.38 172.212 90)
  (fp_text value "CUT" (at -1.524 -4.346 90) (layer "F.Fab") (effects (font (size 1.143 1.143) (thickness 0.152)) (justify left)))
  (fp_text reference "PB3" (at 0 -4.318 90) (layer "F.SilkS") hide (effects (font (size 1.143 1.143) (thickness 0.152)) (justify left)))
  (fp_circle (center 0 0) (end 3.85 0) (layer "F.SilkS") (width 0.254))
  (pad 2 thru_hole rect (at 2.15 0 180) (size 3.5 2.5) (layers "*.Cu" "*.Paste" "*.Mask") (drill oval 1 2.2) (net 7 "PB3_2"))
  (pad 1 thru_hole rect (at -2.15 0 180) (size 3.5 2.5) (layers "*.Cu" "*.Paste" "*.Mask") (drill oval 1 2.2) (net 9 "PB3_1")))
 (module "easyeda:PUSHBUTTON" (layer "F.Cu") (at 22.38 196.342 90)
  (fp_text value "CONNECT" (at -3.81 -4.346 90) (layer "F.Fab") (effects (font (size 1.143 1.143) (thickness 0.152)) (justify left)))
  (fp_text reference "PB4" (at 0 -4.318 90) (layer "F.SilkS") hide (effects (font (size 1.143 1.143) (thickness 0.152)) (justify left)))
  (fp_circle (center 0 0) (end 3.85 0) (layer "F.SilkS") (width 0.254))
  (pad 2 thru_hole rect (at 2.15 0 180) (size 3.5 2.5) (layers "*.Cu" "*.Paste" "*.Mask") (drill oval 1 2.2) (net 7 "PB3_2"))
  (pad 1 thru_hole rect (at -2.15 0 180) (size 3.5 2.5) (layers "*.Cu" "*.Paste" "*.Mask") (drill oval 1 2.2) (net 10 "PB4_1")))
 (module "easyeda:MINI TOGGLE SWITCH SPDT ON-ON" (layer "F.Cu") (at 11.08 185.039 90)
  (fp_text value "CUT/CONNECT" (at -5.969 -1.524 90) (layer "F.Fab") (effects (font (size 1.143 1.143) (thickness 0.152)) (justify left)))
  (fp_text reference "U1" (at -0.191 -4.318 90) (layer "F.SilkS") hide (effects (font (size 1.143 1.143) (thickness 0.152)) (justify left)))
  (fp_line (start -6.604 -3.81) (end 6.396 -3.81) (width 0.254) (layer "F.SilkS") (status 40000))
  (fp_line (start 6.396 -3.81) (end 6.396 4.19) (width 0.254) (layer "F.SilkS") (status 40000))
  (fp_line (start 6.396 4.19) (end -6.604 4.19) (width 0.254) (layer "F.SilkS") (status 40000))
  (fp_line (start -6.604 4.19) (end -6.604 -3.81) (width 0.254) (layer "F.SilkS") (status 40000))
  (pad 2 thru_hole oval (at -4.445 0 90) (size 2 3.3) (layers "*.Cu" "*.Paste" "*.Mask") (drill oval 1.2 2.5) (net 9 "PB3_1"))
  (pad 1 thru_hole oval (at 0 0 90) (size 2 3.3) (layers "*.Cu" "*.Paste" "*.Mask") (drill oval 1.2 2.5) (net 13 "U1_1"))
  (pad 3 thru_hole oval (at 4.445 0 90) (size 2 3.3) (layers "*.Cu" "*.Paste" "*.Mask") (drill oval 1.2 2.5) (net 10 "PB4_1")))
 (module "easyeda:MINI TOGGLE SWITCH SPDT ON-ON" (layer "F.Cu") (at 10.08 135.382 90)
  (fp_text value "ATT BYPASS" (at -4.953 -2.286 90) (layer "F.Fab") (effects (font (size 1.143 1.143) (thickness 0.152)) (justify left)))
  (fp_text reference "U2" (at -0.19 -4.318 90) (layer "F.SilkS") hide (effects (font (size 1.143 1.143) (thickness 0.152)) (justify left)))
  (fp_line (start -6.604 -3.81) (end 6.396 -3.81) (width 0.254) (layer "F.SilkS") (status 40000))
  (fp_line (start 6.396 -3.81) (end 6.396 4.19) (width 0.254) (layer "F.SilkS") (status 40000))
  (fp_line (start 6.396 4.19) (end -6.604 4.19) (width 0.254) (layer "F.SilkS") (status 40000))
  (fp_line (start -6.604 4.19) (end -6.604 -3.81) (width 0.254) (layer "F.SilkS") (status 40000))
  (pad 2 thru_hole oval (at -4.445 0 90) (size 2 3.3) (layers "*.Cu" "*.Paste" "*.Mask") (drill oval 1.2 2.5) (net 6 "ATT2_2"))
  (pad 1 thru_hole oval (at 0 0 90) (size 2 3.3) (layers "*.Cu" "*.Paste" "*.Mask") (drill oval 1.2 2.5) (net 14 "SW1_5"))
  (pad 3 thru_hole oval (at 4.445 0 90) (size 2 3.3) (layers "*.Cu" "*.Paste" "*.Mask") (drill oval 1.2 2.5) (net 7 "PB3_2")))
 (via (at 5.691 215.295) (size 0.8) (drill 0.305) (layers "F.Cu" "B.Cu") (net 3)))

